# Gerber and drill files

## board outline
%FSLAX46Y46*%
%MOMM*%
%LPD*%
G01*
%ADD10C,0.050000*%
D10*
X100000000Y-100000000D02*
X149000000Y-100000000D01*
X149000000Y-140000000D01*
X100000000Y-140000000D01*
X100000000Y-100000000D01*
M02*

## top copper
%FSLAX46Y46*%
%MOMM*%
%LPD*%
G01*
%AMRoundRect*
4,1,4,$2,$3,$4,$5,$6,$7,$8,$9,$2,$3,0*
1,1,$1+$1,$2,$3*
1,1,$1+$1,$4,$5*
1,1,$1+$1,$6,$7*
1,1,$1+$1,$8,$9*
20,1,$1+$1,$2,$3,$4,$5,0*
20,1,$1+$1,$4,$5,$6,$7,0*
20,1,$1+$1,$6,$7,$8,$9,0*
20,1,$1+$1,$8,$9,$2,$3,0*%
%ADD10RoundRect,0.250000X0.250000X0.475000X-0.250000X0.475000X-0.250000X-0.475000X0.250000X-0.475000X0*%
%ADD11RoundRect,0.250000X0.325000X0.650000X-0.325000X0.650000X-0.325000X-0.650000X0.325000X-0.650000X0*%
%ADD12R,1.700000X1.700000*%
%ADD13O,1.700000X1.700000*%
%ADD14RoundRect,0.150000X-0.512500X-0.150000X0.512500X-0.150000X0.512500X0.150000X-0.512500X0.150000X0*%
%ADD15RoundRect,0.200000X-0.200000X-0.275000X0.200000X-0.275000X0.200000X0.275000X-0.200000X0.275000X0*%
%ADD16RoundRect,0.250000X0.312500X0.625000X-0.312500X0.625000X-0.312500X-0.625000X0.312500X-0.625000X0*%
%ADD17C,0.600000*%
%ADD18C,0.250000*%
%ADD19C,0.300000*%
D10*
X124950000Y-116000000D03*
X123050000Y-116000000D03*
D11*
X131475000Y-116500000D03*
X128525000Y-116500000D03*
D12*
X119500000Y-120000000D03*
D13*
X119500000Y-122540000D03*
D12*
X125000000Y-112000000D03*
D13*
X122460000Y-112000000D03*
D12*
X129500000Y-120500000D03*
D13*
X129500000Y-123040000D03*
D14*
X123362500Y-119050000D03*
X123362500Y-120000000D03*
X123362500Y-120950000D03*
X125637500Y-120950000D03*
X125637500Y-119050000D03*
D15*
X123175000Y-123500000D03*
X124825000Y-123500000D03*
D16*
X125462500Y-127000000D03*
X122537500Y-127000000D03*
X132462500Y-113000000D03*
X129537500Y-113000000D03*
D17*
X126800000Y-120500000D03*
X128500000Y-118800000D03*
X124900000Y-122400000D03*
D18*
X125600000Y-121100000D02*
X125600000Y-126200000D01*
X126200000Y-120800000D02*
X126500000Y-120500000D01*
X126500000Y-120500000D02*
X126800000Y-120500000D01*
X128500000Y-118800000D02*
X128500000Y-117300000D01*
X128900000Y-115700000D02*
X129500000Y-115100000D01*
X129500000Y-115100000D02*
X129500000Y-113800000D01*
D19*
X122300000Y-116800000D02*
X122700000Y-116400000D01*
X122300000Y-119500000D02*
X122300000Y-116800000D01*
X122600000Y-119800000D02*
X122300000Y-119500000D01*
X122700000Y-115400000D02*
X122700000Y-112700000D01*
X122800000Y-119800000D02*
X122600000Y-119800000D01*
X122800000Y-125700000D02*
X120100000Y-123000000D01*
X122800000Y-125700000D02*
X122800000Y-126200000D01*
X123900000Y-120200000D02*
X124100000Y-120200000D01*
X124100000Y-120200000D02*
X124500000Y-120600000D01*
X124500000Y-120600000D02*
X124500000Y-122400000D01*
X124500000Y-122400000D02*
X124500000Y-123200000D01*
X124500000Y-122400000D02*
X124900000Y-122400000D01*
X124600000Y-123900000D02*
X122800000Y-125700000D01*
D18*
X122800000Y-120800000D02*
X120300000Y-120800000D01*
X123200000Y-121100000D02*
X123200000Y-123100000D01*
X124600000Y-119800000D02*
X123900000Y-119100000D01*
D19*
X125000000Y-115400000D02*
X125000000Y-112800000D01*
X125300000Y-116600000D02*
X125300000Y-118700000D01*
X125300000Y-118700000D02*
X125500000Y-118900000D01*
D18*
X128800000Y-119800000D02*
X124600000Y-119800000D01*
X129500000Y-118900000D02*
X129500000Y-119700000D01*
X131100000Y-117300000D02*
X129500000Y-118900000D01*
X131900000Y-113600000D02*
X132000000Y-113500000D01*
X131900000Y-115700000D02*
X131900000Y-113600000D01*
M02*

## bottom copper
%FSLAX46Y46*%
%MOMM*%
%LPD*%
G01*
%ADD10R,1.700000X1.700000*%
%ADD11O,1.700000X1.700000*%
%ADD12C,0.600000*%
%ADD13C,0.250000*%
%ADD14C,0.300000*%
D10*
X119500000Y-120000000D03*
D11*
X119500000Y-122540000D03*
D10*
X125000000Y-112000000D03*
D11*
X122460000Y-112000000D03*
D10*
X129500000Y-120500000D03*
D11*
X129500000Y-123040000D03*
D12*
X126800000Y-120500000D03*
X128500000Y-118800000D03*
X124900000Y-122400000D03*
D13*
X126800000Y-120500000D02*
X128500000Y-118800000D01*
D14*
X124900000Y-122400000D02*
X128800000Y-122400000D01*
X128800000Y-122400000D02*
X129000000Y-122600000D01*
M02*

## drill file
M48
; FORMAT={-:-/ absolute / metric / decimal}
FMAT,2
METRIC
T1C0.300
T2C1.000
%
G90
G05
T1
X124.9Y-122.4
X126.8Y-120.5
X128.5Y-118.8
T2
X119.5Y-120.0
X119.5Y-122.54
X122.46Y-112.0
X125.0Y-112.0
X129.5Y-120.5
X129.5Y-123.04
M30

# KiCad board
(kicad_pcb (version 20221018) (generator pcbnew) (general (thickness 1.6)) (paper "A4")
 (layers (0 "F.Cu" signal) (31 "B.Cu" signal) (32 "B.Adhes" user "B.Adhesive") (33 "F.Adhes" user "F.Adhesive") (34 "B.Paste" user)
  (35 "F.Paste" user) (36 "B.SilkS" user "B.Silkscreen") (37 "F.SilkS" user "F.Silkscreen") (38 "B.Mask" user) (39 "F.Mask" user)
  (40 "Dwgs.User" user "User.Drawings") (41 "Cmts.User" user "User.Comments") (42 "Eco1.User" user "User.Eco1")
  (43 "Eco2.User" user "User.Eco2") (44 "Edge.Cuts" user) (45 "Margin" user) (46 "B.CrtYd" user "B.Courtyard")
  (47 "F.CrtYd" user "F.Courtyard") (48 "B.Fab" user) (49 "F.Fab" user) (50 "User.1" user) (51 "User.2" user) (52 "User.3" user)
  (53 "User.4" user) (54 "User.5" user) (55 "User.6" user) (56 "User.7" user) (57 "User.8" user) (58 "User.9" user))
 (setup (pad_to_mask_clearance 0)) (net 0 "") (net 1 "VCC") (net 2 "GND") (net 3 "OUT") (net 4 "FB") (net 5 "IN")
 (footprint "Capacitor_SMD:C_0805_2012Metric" (layer "F.Cu") (at 124 116 180)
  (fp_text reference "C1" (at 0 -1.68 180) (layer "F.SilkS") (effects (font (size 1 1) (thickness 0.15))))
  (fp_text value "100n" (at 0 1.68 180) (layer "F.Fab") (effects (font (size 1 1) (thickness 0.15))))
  (pad "1" smd roundrect (at -0.95 0 180) (size 1 1.45) (layers "F.Cu" "F.Paste" "F.Mask") (roundrect_rratio 0.25) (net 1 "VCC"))
  (pad "2" smd roundrect (at 0.95 0 180) (size 1 1.45) (layers "F.Cu" "F.Paste" "F.Mask") (roundrect_rratio 0.25) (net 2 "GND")))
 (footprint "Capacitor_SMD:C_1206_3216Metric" (layer "F.Cu") (at 130 116.5 180)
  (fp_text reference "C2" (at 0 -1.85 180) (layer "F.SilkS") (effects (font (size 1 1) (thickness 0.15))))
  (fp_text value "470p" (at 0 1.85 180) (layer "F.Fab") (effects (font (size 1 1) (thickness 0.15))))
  (pad "1" smd roundrect (at -1.475 0 180) (size 1.15 1.8) (layers "F.Cu" "F.Paste" "F.Mask") (roundrect_rratio 0.217391) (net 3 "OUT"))
  (pad "2" smd roundrect (at 1.475 0 180) (size 1.15 1.8) (layers "F.Cu" "F.Paste" "F.Mask") (roundrect_rratio 0.217391) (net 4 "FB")))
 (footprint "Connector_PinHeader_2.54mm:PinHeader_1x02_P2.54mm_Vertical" (layer "F.Cu") (at 119.5 120)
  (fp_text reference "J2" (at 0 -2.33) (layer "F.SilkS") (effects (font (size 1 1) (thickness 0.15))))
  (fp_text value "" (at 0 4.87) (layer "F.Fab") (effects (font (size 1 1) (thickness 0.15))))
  (pad "1" thru_hole rect (at 0 0) (size 1.7 1.7) (drill 1) (layers "*.Cu" "*.Mask") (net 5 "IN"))
  (pad "2" thru_hole oval (at 0 2.54) (size 1.7 1.7) (drill 1) (layers "*.Cu" "*.Mask") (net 2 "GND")))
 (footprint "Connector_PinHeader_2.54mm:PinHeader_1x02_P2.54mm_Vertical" (layer "F.Cu") (at 125 112 -90)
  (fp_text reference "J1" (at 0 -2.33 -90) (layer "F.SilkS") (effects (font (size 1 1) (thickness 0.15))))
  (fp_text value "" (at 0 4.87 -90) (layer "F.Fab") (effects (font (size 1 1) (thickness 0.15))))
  (pad "1" thru_hole rect (at 0 0 270) (size 1.7 1.7) (drill 1) (layers "*.Cu" "*.Mask") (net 1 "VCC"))
  (pad "2" thru_hole oval (at 0 2.54 270) (size 1.7 1.7) (drill 1) (layers "*.Cu" "*.Mask") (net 2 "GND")))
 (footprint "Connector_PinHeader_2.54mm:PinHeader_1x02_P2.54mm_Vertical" (layer "F.Cu") (at 129.5 120.5)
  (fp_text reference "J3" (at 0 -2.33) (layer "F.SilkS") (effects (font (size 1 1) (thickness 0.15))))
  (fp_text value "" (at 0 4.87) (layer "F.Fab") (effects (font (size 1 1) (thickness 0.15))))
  (pad "1" thru_hole rect (at 0 0) (size 1.7 1.7) (drill 1) (layers "*.Cu" "*.Mask") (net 3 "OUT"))
  (pad "2" thru_hole oval (at 0 2.54) (size 1.7 1.7) (drill 1) (layers "*.Cu" "*.Mask") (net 2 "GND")))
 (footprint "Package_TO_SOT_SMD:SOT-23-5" (layer "F.Cu") (at 124.5 120)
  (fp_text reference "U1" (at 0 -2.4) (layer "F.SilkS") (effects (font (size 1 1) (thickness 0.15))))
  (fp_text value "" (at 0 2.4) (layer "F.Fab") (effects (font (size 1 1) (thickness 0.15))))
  (pad "1" smd roundrect (at -1.1375 -0.95) (size 1.325 0.6) (layers "F.Cu" "F.Paste" "F.Mask") (roundrect_rratio 0.25) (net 3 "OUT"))
  (pad "2" smd roundrect (at -1.1375 0) (size 1.325 0.6) (layers "F.Cu" "F.Paste" "F.Mask") (roundrect_rratio 0.25) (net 2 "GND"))
  (pad "3" smd roundrect (at -1.1375 0.95) (size 1.325 0.6) (layers "F.Cu" "F.Paste" "F.Mask") (roundrect_rratio 0.25) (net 5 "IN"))
  (pad "4" smd roundrect (at 1.1375 0.95) (size 1.325 0.6) (layers "F.Cu" "F.Paste" "F.Mask") (roundrect_rratio 0.25) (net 4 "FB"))
  (pad "5" smd roundrect (at 1.1375 -0.95) (size 1.325 0.6) (layers "F.Cu" "F.Paste" "F.Mask") (roundrect_rratio 0.25) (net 1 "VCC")))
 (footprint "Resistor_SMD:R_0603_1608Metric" (layer "F.Cu") (at 124 123.5)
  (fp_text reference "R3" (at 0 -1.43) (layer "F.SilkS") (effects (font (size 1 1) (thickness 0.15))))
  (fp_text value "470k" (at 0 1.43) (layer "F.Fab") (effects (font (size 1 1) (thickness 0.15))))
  (pad "1" smd roundrect (at -0.825 0) (size 0.8 0.95) (layers "F.Cu" "F.Paste" "F.Mask") (roundrect_rratio 0.25) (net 5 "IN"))
  (pad "2" smd roundrect (at 0.825 0) (size 0.8 0.95) (layers "F.Cu" "F.Paste" "F.Mask") (roundrect_rratio 0.25) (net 2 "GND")))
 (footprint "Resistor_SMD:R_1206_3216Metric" (layer "F.Cu") (at 124 127 180)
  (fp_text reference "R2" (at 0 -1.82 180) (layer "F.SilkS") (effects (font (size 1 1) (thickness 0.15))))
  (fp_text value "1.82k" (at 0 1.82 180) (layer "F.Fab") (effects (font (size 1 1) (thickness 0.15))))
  (pad "1" smd roundrect (at -1.4625 0 180) (size 1.125 1.75) (layers "F.Cu" "F.Paste" "F.Mask") (roundrect_rratio 0.222222) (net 4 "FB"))
  (pad "2" smd roundrect (at 1.4625 0 180) (size 1.125 1.75) (layers "F.Cu" "F.Paste" "F.Mask") (roundrect_rratio 0.222222) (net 2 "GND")))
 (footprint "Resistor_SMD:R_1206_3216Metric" (layer "F.Cu") (at 131 113 180)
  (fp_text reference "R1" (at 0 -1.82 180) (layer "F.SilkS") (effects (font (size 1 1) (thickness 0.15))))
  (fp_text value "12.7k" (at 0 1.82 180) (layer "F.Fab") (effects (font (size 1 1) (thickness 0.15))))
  (pad "1" smd roundrect (at -1.4625 0 180) (size 1.125 1.75) (layers "F.Cu" "F.Paste" "F.Mask") (roundrect_rratio 0.222222) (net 3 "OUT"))
  (pad "2" smd roundrect (at 1.4625 0 180) (size 1.125 1.75) (layers "F.Cu" "F.Paste" "F.Mask") (roundrect_rratio 0.222222) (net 4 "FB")))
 (gr_rect (start 100 100) (end 149 140) (stroke (width 0.05) (type default)) (fill none) (layer "Edge.Cuts"))
 (segment (start 125.6 121.1) (end 125.6 126.2) (width 0.25) (layer "F.Cu") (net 4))
 (segment (start 126.2 120.8) (end 126.5 120.5) (width 0.25) (layer "F.Cu") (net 4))
 (segment (start 126.5 120.5) (end 126.8 120.5) (width 0.25) (layer "F.Cu") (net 4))
 (segment (start 128.5 118.8) (end 128.5 117.3) (width 0.25) (layer "F.Cu") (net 4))
 (segment (start 128.9 115.7) (end 129.5 115.1) (width 0.25) (layer "F.Cu") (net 4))
 (segment (start 129.5 115.1) (end 129.5 113.8) (width 0.25) (layer "F.Cu") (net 4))
 (via (at 126.8 120.5) (size 0.6) (drill 0.3) (layers "F.Cu" "B.Cu") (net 4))
 (via (at 128.5 118.8) (size 0.6) (drill 0.3) (layers "F.Cu" "B.Cu") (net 4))
 (segment (start 122.3 116.8) (end 122.7 116.4) (width 0.3) (layer "F.Cu") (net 2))
 (segment (start 122.3 119.5) (end 122.3 116.8) (width 0.3) (layer "F.Cu") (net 2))
 (segment (start 122.6 119.8) (end 122.3 119.5) (width 0.3) (layer "F.Cu") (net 2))
 (segment (start 122.7 115.4) (end 122.7 112.7) (width 0.3) (layer "F.Cu") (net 2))
 (segment (start 122.8 119.8) (end 122.6 119.8) (width 0.3) (layer "F.Cu") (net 2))
 (segment (start 122.8 125.7) (end 120.1 123) (width 0.3) (layer "F.Cu") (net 2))
 (segment (start 122.8 125.7) (end 122.8 126.2) (width 0.3) (layer "F.Cu") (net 2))
 (segment (start 123.9 120.2) (end 124.1 120.2) (width 0.3) (layer "F.Cu") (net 2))
 (segment (start 124.1 120.2) (end 124.5 120.6) (width 0.3) (layer "F.Cu") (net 2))
 (segment (start 124.5 120.6) (end 124.5 122.4) (width 0.3) (layer "F.Cu") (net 2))
 (segment (start 124.5 122.4) (end 124.5 123.2) (width 0.3) (layer "F.Cu") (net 2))
 (segment (start 124.5 122.4) (end 124.9 122.4) (width 0.3) (layer "F.Cu") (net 2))
 (segment (start 124.6 123.9) (end 122.8 125.7) (width 0.3) (layer "F.Cu") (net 2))
 (segment (start 126.8 120.5) (end 128.5 118.8) (width 0.25) (layer "B.Cu") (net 4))
 (via (at 124.9 122.4) (size 0.6) (drill 0.3) (layers "F.Cu" "B.Cu") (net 2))
 (segment (start 122.8 120.8) (end 120.3 120.8) (width 0.25) (layer "F.Cu") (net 5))
 (segment (start 123.2 121.1) (end 123.2 123.1) (width 0.25) (layer "F.Cu") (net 5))
 (segment (start 124.6 119.8) (end 123.9 119.1) (width 0.25) (layer "F.Cu") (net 3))
 (segment (start 124.9 122.4) (end 128.8 122.4) (width 0.3) (layer "B.Cu") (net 2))
 (segment (start 125 115.4) (end 125 112.8) (width 0.3) (layer "F.Cu") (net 1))
 (segment (start 125.3 116.6) (end 125.3 118.7) (width 0.3) (layer "F.Cu") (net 1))
 (segment (start 125.3 118.7) (end 125.5 118.9) (width 0.3) (layer "F.Cu") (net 1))
 (segment (start 128.8 119.8) (end 124.6 119.8) (width 0.25) (layer "F.Cu") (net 3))
 (segment (start 128.8 122.4) (end 129 122.6) (width 0.3) (layer "B.Cu") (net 2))
 (segment (start 129.5 118.9) (end 129.5 119.7) (width 0.25) (layer "F.Cu") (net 3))
 (segment (start 131.1 117.3) (end 129.5 118.9) (width 0.25) (layer "F.Cu") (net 3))
 (segment (start 131.9 113.6) (end 132 113.5) (width 0.25) (layer "F.Cu") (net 3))
 (segment (start 131.9 115.7) (end 131.9 113.6) (width 0.25) (layer "F.Cu") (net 3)))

